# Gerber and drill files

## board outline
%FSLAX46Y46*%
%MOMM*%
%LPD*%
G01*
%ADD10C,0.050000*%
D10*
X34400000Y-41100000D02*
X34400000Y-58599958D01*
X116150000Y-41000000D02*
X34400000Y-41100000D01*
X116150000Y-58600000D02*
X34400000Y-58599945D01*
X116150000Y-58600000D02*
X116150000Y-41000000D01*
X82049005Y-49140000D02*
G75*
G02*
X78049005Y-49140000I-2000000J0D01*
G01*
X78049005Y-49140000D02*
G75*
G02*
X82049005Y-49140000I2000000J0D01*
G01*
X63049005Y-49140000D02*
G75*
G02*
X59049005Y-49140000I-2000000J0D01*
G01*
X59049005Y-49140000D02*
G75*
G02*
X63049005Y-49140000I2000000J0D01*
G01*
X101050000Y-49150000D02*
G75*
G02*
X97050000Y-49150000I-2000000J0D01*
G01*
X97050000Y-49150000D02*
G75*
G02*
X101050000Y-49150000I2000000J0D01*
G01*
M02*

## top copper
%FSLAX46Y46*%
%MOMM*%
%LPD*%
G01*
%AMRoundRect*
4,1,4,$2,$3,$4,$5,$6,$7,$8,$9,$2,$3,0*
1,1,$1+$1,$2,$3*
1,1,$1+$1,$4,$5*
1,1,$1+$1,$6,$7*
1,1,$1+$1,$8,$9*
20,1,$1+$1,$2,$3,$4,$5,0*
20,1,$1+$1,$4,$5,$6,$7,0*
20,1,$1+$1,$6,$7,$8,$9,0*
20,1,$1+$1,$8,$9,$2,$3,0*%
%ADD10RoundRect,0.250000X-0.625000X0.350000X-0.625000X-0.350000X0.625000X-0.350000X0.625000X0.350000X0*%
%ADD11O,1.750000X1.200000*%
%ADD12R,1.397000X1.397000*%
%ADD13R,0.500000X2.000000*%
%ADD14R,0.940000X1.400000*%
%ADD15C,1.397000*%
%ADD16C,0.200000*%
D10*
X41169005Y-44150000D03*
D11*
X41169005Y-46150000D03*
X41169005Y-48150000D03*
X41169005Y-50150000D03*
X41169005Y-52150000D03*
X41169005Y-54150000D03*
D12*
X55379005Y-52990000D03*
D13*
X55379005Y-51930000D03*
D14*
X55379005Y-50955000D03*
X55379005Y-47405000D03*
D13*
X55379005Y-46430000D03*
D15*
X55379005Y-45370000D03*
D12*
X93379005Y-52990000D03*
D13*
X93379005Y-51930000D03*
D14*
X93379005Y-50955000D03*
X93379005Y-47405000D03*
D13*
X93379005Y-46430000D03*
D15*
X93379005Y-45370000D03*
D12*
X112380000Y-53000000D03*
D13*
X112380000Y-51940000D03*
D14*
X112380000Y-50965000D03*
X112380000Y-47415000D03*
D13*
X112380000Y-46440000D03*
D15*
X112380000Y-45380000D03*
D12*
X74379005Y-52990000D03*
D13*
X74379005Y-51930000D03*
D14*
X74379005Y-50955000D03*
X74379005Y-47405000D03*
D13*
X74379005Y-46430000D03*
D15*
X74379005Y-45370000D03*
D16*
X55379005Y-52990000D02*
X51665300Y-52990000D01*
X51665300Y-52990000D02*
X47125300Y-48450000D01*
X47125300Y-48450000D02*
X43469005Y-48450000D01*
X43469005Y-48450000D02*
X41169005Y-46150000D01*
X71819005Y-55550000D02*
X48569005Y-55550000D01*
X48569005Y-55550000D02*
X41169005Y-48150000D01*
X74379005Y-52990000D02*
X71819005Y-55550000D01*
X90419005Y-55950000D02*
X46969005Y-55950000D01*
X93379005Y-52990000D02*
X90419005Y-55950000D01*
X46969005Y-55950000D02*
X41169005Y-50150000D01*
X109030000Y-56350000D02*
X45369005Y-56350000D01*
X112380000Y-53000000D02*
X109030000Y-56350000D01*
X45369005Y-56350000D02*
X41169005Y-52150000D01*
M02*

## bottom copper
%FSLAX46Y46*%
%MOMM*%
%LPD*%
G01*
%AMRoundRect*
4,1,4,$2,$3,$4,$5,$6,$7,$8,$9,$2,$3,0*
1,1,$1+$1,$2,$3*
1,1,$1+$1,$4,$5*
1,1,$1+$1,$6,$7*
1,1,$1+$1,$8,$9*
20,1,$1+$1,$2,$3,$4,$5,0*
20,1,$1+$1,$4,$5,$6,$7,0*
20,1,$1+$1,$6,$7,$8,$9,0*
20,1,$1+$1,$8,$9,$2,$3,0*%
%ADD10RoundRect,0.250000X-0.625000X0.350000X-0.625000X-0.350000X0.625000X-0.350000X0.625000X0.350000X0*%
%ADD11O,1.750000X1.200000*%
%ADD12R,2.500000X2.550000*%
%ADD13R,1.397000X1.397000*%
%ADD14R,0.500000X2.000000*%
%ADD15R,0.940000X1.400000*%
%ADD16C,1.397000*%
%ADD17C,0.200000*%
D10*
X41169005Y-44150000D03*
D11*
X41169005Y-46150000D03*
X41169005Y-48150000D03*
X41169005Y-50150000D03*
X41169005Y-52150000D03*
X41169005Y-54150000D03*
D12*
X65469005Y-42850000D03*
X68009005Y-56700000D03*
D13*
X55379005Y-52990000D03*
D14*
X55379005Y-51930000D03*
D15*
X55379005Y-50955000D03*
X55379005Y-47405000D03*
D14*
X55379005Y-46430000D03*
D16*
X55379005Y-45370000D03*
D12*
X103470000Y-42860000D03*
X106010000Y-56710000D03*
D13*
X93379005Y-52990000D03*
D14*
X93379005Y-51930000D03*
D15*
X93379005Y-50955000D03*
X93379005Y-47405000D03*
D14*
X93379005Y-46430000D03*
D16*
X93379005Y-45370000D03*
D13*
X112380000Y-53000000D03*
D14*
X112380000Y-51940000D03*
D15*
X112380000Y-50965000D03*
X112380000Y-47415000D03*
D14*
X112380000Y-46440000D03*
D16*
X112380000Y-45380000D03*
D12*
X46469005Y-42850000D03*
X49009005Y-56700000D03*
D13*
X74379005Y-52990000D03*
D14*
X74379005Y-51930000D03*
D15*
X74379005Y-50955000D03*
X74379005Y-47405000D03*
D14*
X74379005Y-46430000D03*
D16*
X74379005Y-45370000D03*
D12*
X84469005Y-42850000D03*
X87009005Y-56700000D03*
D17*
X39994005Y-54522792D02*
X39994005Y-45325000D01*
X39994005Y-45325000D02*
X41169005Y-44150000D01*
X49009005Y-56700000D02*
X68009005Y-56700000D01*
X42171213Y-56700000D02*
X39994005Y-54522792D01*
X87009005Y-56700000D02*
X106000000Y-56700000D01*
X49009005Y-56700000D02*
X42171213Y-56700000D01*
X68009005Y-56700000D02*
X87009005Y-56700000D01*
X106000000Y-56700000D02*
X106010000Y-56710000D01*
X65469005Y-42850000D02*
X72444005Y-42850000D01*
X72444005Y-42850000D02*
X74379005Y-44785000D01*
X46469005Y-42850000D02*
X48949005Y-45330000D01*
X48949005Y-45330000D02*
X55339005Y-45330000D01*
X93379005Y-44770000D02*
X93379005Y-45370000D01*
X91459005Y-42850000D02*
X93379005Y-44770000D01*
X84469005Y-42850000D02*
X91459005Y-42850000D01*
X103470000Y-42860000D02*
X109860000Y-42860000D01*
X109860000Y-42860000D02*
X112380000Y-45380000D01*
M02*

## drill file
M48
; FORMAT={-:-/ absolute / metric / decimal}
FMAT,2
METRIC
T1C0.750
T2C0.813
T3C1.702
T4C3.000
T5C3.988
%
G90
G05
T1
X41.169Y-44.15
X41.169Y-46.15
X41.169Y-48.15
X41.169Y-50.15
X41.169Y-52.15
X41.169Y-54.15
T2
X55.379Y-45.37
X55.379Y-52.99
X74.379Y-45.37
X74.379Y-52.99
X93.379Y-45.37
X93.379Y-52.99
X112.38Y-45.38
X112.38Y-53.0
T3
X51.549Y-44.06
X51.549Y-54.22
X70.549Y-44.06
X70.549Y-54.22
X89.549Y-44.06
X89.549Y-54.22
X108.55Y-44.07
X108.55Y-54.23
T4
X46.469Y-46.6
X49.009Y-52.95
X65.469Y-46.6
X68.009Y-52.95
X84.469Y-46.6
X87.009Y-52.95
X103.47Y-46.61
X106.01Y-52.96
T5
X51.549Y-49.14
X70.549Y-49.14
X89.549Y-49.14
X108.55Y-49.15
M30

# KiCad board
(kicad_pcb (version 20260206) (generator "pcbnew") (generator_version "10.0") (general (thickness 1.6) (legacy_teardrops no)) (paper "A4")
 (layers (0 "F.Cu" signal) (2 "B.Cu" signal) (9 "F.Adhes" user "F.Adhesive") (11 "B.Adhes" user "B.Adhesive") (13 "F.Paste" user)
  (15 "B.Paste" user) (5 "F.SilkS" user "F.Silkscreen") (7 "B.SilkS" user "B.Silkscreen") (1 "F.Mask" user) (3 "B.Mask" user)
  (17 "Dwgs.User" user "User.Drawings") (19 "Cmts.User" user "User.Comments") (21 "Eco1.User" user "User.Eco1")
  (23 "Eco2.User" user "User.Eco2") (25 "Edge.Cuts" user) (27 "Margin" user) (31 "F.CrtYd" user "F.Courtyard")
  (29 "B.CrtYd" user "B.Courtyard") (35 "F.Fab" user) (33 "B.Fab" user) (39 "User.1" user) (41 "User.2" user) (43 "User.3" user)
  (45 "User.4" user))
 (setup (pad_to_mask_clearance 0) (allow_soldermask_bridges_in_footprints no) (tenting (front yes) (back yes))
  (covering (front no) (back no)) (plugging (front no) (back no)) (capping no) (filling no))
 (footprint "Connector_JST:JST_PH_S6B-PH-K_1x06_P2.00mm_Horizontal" (layer "F.Cu") (at 41.169005 44.15 -90)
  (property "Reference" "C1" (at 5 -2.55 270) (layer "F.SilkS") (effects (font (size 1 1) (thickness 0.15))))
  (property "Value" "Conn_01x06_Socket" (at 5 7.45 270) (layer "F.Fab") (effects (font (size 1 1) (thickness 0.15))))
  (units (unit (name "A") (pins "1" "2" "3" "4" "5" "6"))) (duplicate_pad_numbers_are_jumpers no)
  (pad "1" thru_hole roundrect (at 0 0 270) (size 1.2 1.75) (drill 0.75) (layers "*.Cu" "*.Mask") (remove_unused_layers no)
   (roundrect_rratio 0.208333) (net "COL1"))
  (pad "2" thru_hole oval (at 2 0 270) (size 1.2 1.75) (drill 0.75) (layers "*.Cu" "*.Mask") (remove_unused_layers no) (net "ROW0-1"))
  (pad "3" thru_hole oval (at 4 0 270) (size 1.2 1.75) (drill 0.75) (layers "*.Cu" "*.Mask") (remove_unused_layers no) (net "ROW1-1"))
  (pad "4" thru_hole oval (at 6 0 270) (size 1.2 1.75) (drill 0.75) (layers "*.Cu" "*.Mask") (remove_unused_layers no) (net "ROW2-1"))
  (pad "5" thru_hole oval (at 8 0 270) (size 1.2 1.75) (drill 0.75) (layers "*.Cu" "*.Mask") (remove_unused_layers no) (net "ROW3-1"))
  (pad "6" thru_hole oval (at 10 0 270) (size 1.2 1.75) (drill 0.75) (layers "*.Cu" "*.Mask") (remove_unused_layers no) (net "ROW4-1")))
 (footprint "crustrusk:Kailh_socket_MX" (layer "F.Cu") (at 70.549005 49.14 90)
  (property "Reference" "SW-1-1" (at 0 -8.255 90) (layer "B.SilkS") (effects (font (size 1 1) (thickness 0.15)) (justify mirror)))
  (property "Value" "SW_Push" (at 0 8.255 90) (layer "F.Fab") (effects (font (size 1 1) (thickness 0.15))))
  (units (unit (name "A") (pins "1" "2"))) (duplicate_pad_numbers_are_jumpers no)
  (pad "" np_thru_hole circle (at -5.08 0 90) (size 1.7018 1.7018) (drill 1.7018) (layers "*.Cu" "*.Mask"))
  (pad "" np_thru_hole circle (at -3.81 -2.54 90) (size 3 3) (drill 3) (layers "*.Cu" "*.Mask"))
  (pad "" np_thru_hole circle (at 0 0 90) (size 3.9878 3.9878) (drill 3.9878) (layers "*.Cu" "*.Mask"))
  (pad "" np_thru_hole circle (at 2.54 -5.08 90) (size 3 3) (drill 3) (layers "*.Cu" "*.Mask"))
  (pad "" np_thru_hole circle (at 5.08 0 90) (size 1.7018 1.7018) (drill 1.7018) (layers "*.Cu" "*.Mask"))
  (pad "1" smd rect (at 6.29 -5.08 90) (size 2.55 2.5) (layers "B.Cu" "B.Mask" "B.Paste") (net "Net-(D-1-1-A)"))
  (pad "2" smd rect (at -7.56 -2.54 90) (size 2.55 2.5) (layers "B.Cu" "B.Mask" "B.Paste") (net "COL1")))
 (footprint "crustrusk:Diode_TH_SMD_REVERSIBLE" (layer "F.Cu") (at 55.379005 49.18 90)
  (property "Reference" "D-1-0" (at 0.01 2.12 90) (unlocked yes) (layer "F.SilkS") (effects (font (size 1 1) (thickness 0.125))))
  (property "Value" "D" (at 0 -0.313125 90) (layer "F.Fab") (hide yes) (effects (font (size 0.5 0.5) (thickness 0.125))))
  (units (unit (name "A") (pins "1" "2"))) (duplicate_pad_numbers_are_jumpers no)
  (pad "1" thru_hole rect (at -3.81 0 90) (size 1.397 1.397) (drill 0.8128) (layers "*.Cu" "*.Mask") (remove_unused_layers no)
   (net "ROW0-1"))
  (pad "1" smd rect (at -2.75 0 270) (size 2 0.5) (layers "F.Cu") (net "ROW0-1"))
  (pad "1" smd rect (at -2.75 0 90) (size 2 0.5) (layers "B.Cu") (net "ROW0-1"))
  (pad "1" smd rect (at -1.775 0 270) (size 1.4 0.94) (layers "F.Cu" "F.Mask" "F.Paste") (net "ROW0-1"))
  (pad "1" smd rect (at -1.775 0 90) (size 1.4 0.94) (layers "B.Cu" "B.Mask" "B.Paste") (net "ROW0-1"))
  (pad "2" smd rect (at 1.775 0 270) (size 1.4 0.94) (layers "F.Cu" "F.Mask" "F.Paste") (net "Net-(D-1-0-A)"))
  (pad "2" smd rect (at 1.775 0 90) (size 1.4 0.94) (layers "B.Cu" "B.Mask" "B.Paste") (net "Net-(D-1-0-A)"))
  (pad "2" smd rect (at 2.75 0 270) (size 2 0.5) (layers "F.Cu") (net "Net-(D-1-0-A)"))
  (pad "2" smd rect (at 2.75 0 90) (size 2 0.5) (layers "B.Cu") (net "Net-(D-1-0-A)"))
  (pad "2" thru_hole circle (at 3.81 0 90) (size 1.397 1.397) (drill 0.8128) (layers "*.Cu" "*.Mask") (remove_unused_layers no)
   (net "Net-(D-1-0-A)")))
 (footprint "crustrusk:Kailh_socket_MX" (layer "F.Cu") (at 108.55 49.15 90)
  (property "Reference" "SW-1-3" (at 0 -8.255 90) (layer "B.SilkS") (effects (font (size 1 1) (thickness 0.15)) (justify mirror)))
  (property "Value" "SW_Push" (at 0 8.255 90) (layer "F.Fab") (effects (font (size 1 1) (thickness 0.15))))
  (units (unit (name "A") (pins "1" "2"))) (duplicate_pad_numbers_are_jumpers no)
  (pad "" np_thru_hole circle (at -5.08 0 90) (size 1.7018 1.7018) (drill 1.7018) (layers "*.Cu" "*.Mask"))
  (pad "" np_thru_hole circle (at -3.81 -2.54 90) (size 3 3) (drill 3) (layers "*.Cu" "*.Mask"))
  (pad "" np_thru_hole circle (at 0 0 90) (size 3.9878 3.9878) (drill 3.9878) (layers "*.Cu" "*.Mask"))
  (pad "" np_thru_hole circle (at 2.54 -5.08 90) (size 3 3) (drill 3) (layers "*.Cu" "*.Mask"))
  (pad "" np_thru_hole circle (at 5.08 0 90) (size 1.7018 1.7018) (drill 1.7018) (layers "*.Cu" "*.Mask"))
  (pad "1" smd rect (at 6.29 -5.08 90) (size 2.55 2.5) (layers "B.Cu" "B.Mask" "B.Paste") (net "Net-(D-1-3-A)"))
  (pad "2" smd rect (at -7.56 -2.54 90) (size 2.55 2.5) (layers "B.Cu" "B.Mask" "B.Paste") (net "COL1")))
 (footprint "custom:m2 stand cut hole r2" (layer "F.Cu") (at 80.049005 49.14 90)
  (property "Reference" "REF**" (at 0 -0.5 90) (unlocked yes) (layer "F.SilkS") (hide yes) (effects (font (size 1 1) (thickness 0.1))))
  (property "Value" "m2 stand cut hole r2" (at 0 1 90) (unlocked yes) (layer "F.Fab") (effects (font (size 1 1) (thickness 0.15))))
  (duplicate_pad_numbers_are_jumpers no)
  (fp_circle (center 0 0) (end 2 0) (stroke (width 0.05) (type default)) (fill no) (layer "Edge.Cuts")))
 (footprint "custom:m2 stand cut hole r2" (layer "F.Cu") (at 61.049005 49.14 90)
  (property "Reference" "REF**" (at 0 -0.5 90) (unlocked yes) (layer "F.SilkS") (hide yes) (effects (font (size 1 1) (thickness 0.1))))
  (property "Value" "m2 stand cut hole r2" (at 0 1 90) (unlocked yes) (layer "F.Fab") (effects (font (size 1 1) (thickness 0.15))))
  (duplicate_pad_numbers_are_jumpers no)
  (fp_circle (center 0 0) (end 2 0) (stroke (width 0.05) (type default)) (fill no) (layer "Edge.Cuts")))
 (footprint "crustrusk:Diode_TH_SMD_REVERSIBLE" (layer "F.Cu") (at 93.379005 49.18 90)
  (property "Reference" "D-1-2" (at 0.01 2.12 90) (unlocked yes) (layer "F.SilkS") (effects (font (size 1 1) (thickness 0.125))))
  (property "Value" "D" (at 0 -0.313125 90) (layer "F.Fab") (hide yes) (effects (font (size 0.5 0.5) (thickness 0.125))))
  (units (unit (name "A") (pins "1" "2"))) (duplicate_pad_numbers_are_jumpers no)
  (pad "1" thru_hole rect (at -3.81 0 90) (size 1.397 1.397) (drill 0.8128) (layers "*.Cu" "*.Mask") (remove_unused_layers no)
   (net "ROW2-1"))
  (pad "1" smd rect (at -2.75 0 270) (size 2 0.5) (layers "F.Cu") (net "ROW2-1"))
  (pad "1" smd rect (at -2.75 0 90) (size 2 0.5) (layers "B.Cu") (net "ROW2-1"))
  (pad "1" smd rect (at -1.775 0 270) (size 1.4 0.94) (layers "F.Cu" "F.Mask" "F.Paste") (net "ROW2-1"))
  (pad "1" smd rect (at -1.775 0 90) (size 1.4 0.94) (layers "B.Cu" "B.Mask" "B.Paste") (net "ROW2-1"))
  (pad "2" smd rect (at 1.775 0 270) (size 1.4 0.94) (layers "F.Cu" "F.Mask" "F.Paste") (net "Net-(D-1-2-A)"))
  (pad "2" smd rect (at 1.775 0 90) (size 1.4 0.94) (layers "B.Cu" "B.Mask" "B.Paste") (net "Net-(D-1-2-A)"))
  (pad "2" smd rect (at 2.75 0 270) (size 2 0.5) (layers "F.Cu") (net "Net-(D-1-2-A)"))
  (pad "2" smd rect (at 2.75 0 90) (size 2 0.5) (layers "B.Cu") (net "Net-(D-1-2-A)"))
  (pad "2" thru_hole circle (at 3.81 0 90) (size 1.397 1.397) (drill 0.8128) (layers "*.Cu" "*.Mask") (remove_unused_layers no)
   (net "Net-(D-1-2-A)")))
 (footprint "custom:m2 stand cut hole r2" (layer "F.Cu") (at 99.05 49.15 90)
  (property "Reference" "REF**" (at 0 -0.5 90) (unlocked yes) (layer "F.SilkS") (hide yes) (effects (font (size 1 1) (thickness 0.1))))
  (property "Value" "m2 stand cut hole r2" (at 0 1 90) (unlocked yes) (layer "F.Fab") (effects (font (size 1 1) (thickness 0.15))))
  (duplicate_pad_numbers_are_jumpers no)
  (fp_circle (center 0 0) (end 2 0) (stroke (width 0.05) (type default)) (fill no) (layer "Edge.Cuts")))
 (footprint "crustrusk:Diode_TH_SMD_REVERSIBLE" (layer "F.Cu") (at 112.38 49.19 90)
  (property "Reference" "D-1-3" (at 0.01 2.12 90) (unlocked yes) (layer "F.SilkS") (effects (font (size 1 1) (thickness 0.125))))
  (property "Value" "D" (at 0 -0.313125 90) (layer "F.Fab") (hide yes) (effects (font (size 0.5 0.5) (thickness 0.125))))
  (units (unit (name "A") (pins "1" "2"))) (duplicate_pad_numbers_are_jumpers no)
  (pad "1" thru_hole rect (at -3.81 0 90) (size 1.397 1.397) (drill 0.8128) (layers "*.Cu" "*.Mask") (remove_unused_layers no)
   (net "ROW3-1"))
  (pad "1" smd rect (at -2.75 0 270) (size 2 0.5) (layers "F.Cu") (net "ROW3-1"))
  (pad "1" smd rect (at -2.75 0 90) (size 2 0.5) (layers "B.Cu") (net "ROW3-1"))
  (pad "1" smd rect (at -1.775 0 270) (size 1.4 0.94) (layers "F.Cu" "F.Mask" "F.Paste") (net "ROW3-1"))
  (pad "1" smd rect (at -1.775 0 90) (size 1.4 0.94) (layers "B.Cu" "B.Mask" "B.Paste") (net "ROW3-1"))
  (pad "2" smd rect (at 1.775 0 270) (size 1.4 0.94) (layers "F.Cu" "F.Mask" "F.Paste") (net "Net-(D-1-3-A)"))
  (pad "2" smd rect (at 1.775 0 90) (size 1.4 0.94) (layers "B.Cu" "B.Mask" "B.Paste") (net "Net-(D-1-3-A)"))
  (pad "2" smd rect (at 2.75 0 270) (size 2 0.5) (layers "F.Cu") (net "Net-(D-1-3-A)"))
  (pad "2" smd rect (at 2.75 0 90) (size 2 0.5) (layers "B.Cu") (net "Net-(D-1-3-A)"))
  (pad "2" thru_hole circle (at 3.81 0 90) (size 1.397 1.397) (drill 0.8128) (layers "*.Cu" "*.Mask") (remove_unused_layers no)
   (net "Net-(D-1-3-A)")))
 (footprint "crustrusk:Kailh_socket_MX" (layer "F.Cu") (at 51.549005 49.14 90)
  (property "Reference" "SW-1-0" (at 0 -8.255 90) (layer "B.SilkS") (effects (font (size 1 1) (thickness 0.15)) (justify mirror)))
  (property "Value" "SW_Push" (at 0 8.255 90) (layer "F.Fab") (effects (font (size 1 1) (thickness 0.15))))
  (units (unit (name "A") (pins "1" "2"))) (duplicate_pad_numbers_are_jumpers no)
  (pad "" np_thru_hole circle (at -5.08 0 90) (size 1.7018 1.7018) (drill 1.7018) (layers "*.Cu" "*.Mask"))
  (pad "" np_thru_hole circle (at -3.81 -2.54 90) (size 3 3) (drill 3) (layers "*.Cu" "*.Mask"))
  (pad "" np_thru_hole circle (at 0 0 90) (size 3.9878 3.9878) (drill 3.9878) (layers "*.Cu" "*.Mask"))
  (pad "" np_thru_hole circle (at 2.54 -5.08 90) (size 3 3) (drill 3) (layers "*.Cu" "*.Mask"))
  (pad "" np_thru_hole circle (at 5.08 0 90) (size 1.7018 1.7018) (drill 1.7018) (layers "*.Cu" "*.Mask"))
  (pad "1" smd rect (at 6.29 -5.08 90) (size 2.55 2.5) (layers "B.Cu" "B.Mask" "B.Paste") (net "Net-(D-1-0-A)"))
  (pad "2" smd rect (at -7.56 -2.54 90) (size 2.55 2.5) (layers "B.Cu" "B.Mask" "B.Paste") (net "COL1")))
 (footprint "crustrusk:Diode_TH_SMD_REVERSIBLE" (layer "F.Cu") (at 74.379005 49.18 90)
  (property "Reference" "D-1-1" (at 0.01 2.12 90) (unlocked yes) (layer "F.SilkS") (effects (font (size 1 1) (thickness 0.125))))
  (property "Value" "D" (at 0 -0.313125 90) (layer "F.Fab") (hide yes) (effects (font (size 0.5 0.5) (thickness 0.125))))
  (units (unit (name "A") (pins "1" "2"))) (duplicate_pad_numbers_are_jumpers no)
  (pad "1" thru_hole rect (at -3.81 0 90) (size 1.397 1.397) (drill 0.8128) (layers "*.Cu" "*.Mask") (remove_unused_layers no)
   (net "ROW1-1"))
  (pad "1" smd rect (at -2.75 0 270) (size 2 0.5) (layers "F.Cu") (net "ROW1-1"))
  (pad "1" smd rect (at -2.75 0 90) (size 2 0.5) (layers "B.Cu") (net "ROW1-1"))
  (pad "1" smd rect (at -1.775 0 270) (size 1.4 0.94) (layers "F.Cu" "F.Mask" "F.Paste") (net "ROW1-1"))
  (pad "1" smd rect (at -1.775 0 90) (size 1.4 0.94) (layers "B.Cu" "B.Mask" "B.Paste") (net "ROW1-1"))
  (pad "2" smd rect (at 1.775 0 270) (size 1.4 0.94) (layers "F.Cu" "F.Mask" "F.Paste") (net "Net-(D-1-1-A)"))
  (pad "2" smd rect (at 1.775 0 90) (size 1.4 0.94) (layers "B.Cu" "B.Mask" "B.Paste") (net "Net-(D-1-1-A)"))
  (pad "2" smd rect (at 2.75 0 270) (size 2 0.5) (layers "F.Cu") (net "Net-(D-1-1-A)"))
  (pad "2" smd rect (at 2.75 0 90) (size 2 0.5) (layers "B.Cu") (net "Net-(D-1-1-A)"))
  (pad "2" thru_hole circle (at 3.81 0 90) (size 1.397 1.397) (drill 0.8128) (layers "*.Cu" "*.Mask") (remove_unused_layers no)
   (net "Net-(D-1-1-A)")))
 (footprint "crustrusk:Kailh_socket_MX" (layer "F.Cu") (at 89.549005 49.14 90)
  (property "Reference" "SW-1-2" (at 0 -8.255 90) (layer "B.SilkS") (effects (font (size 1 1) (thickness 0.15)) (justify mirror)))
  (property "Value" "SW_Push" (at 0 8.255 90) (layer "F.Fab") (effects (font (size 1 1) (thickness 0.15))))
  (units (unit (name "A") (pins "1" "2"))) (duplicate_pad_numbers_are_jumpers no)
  (pad "" np_thru_hole circle (at -5.08 0 90) (size 1.7018 1.7018) (drill 1.7018) (layers "*.Cu" "*.Mask"))
  (pad "" np_thru_hole circle (at -3.81 -2.54 90) (size 3 3) (drill 3) (layers "*.Cu" "*.Mask"))
  (pad "" np_thru_hole circle (at 0 0 90) (size 3.9878 3.9878) (drill 3.9878) (layers "*.Cu" "*.Mask"))
  (pad "" np_thru_hole circle (at 2.54 -5.08 90) (size 3 3) (drill 3) (layers "*.Cu" "*.Mask"))
  (pad "" np_thru_hole circle (at 5.08 0 90) (size 1.7018 1.7018) (drill 1.7018) (layers "*.Cu" "*.Mask"))
  (pad "1" smd rect (at 6.29 -5.08 90) (size 2.55 2.5) (layers "B.Cu" "B.Mask" "B.Paste") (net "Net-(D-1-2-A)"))
  (pad "2" smd rect (at -7.56 -2.54 90) (size 2.55 2.5) (layers "B.Cu" "B.Mask" "B.Paste") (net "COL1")))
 (gr_line (start 34.4 41.1) (end 34.4 58.599958) (stroke (width 0.05) (type default)) (layer "Edge.Cuts"))
 (gr_line (start 116.15 41) (end 34.4 41.1) (stroke (width 0.05) (type default)) (layer "Edge.Cuts"))
 (gr_line (start 116.15 58.6) (end 34.4 58.599945) (stroke (width 0.05) (type default)) (layer "Edge.Cuts"))
 (gr_line (start 116.15 58.6) (end 116.15 41) (stroke (width 0.05) (type default)) (layer "Edge.Cuts"))
 (segment (start 39.994005 54.522792) (end 39.994005 45.325) (width 0.2) (layer "B.Cu") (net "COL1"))
 (segment (start 39.994005 45.325) (end 41.169005 44.15) (width 0.2) (layer "B.Cu") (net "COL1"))
 (segment (start 49.009005 56.7) (end 68.009005 56.7) (width 0.2) (layer "B.Cu") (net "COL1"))
 (segment (start 42.171213 56.7) (end 39.994005 54.522792) (width 0.2) (layer "B.Cu") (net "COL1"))
 (segment (start 87.009005 56.7) (end 106 56.7) (width 0.2) (layer "B.Cu") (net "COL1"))
 (segment (start 49.009005 56.7) (end 42.171213 56.7) (width 0.2) (layer "B.Cu") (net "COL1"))
 (segment (start 68.009005 56.7) (end 87.009005 56.7) (width 0.2) (layer "B.Cu") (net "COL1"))
 (segment (start 106 56.7) (end 106.01 56.71) (width 0.2) (layer "B.Cu") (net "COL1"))
 (segment (start 55.379005 52.99) (end 51.6653 52.99) (width 0.2) (layer "F.Cu") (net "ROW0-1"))
 (segment (start 51.6653 52.99) (end 47.1253 48.45) (width 0.2) (layer "F.Cu") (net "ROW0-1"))
 (segment (start 47.1253 48.45) (end 43.469005 48.45) (width 0.2) (layer "F.Cu") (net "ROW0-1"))
 (segment (start 43.469005 48.45) (end 41.169005 46.15) (width 0.2) (layer "F.Cu") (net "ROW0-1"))
 (segment (start 71.819005 55.55) (end 48.569005 55.55) (width 0.2) (layer "F.Cu") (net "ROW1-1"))
 (segment (start 48.569005 55.55) (end 41.169005 48.15) (width 0.2) (layer "F.Cu") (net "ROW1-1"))
 (segment (start 74.379005 52.99) (end 71.819005 55.55) (width 0.2) (layer "F.Cu") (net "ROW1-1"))
 (segment (start 90.419005 55.95) (end 46.969005 55.95) (width 0.2) (layer "F.Cu") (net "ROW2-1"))
 (segment (start 93.379005 52.99) (end 90.419005 55.95) (width 0.2) (layer "F.Cu") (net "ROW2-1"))
 (segment (start 46.969005 55.95) (end 41.169005 50.15) (width 0.2) (layer "F.Cu") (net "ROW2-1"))
 (segment (start 109.03 56.35) (end 45.369005 56.35) (width 0.2) (layer "F.Cu") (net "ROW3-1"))
 (segment (start 112.38 53) (end 109.03 56.35) (width 0.2) (layer "F.Cu") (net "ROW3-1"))
 (segment (start 45.369005 56.35) (end 41.169005 52.15) (width 0.2) (layer "F.Cu") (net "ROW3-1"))
 (segment (start 65.469005 42.85) (end 72.444005 42.85) (width 0.2) (layer "B.Cu") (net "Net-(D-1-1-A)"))
 (segment (start 72.444005 42.85) (end 74.379005 44.785) (width 0.2) (layer "B.Cu") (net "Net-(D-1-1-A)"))
 (segment (start 46.469005 42.85) (end 48.949005 45.33) (width 0.2) (layer "B.Cu") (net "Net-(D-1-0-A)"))
 (segment (start 48.949005 45.33) (end 55.339005 45.33) (width 0.2) (layer "B.Cu") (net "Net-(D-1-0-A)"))
 (segment (start 93.379005 44.77) (end 93.379005 45.37) (width 0.2) (layer "B.Cu") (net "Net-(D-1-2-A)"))
 (segment (start 91.459005 42.85) (end 93.379005 44.77) (width 0.2) (layer "B.Cu") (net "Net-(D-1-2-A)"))
 (segment (start 84.469005 42.85) (end 91.459005 42.85) (width 0.2) (layer "B.Cu") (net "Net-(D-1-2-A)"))
 (segment (start 103.47 42.86) (end 109.86 42.86) (width 0.2) (layer "B.Cu") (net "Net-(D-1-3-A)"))
 (segment (start 109.86 42.86) (end 112.38 45.38) (width 0.2) (layer "B.Cu") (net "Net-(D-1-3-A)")))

